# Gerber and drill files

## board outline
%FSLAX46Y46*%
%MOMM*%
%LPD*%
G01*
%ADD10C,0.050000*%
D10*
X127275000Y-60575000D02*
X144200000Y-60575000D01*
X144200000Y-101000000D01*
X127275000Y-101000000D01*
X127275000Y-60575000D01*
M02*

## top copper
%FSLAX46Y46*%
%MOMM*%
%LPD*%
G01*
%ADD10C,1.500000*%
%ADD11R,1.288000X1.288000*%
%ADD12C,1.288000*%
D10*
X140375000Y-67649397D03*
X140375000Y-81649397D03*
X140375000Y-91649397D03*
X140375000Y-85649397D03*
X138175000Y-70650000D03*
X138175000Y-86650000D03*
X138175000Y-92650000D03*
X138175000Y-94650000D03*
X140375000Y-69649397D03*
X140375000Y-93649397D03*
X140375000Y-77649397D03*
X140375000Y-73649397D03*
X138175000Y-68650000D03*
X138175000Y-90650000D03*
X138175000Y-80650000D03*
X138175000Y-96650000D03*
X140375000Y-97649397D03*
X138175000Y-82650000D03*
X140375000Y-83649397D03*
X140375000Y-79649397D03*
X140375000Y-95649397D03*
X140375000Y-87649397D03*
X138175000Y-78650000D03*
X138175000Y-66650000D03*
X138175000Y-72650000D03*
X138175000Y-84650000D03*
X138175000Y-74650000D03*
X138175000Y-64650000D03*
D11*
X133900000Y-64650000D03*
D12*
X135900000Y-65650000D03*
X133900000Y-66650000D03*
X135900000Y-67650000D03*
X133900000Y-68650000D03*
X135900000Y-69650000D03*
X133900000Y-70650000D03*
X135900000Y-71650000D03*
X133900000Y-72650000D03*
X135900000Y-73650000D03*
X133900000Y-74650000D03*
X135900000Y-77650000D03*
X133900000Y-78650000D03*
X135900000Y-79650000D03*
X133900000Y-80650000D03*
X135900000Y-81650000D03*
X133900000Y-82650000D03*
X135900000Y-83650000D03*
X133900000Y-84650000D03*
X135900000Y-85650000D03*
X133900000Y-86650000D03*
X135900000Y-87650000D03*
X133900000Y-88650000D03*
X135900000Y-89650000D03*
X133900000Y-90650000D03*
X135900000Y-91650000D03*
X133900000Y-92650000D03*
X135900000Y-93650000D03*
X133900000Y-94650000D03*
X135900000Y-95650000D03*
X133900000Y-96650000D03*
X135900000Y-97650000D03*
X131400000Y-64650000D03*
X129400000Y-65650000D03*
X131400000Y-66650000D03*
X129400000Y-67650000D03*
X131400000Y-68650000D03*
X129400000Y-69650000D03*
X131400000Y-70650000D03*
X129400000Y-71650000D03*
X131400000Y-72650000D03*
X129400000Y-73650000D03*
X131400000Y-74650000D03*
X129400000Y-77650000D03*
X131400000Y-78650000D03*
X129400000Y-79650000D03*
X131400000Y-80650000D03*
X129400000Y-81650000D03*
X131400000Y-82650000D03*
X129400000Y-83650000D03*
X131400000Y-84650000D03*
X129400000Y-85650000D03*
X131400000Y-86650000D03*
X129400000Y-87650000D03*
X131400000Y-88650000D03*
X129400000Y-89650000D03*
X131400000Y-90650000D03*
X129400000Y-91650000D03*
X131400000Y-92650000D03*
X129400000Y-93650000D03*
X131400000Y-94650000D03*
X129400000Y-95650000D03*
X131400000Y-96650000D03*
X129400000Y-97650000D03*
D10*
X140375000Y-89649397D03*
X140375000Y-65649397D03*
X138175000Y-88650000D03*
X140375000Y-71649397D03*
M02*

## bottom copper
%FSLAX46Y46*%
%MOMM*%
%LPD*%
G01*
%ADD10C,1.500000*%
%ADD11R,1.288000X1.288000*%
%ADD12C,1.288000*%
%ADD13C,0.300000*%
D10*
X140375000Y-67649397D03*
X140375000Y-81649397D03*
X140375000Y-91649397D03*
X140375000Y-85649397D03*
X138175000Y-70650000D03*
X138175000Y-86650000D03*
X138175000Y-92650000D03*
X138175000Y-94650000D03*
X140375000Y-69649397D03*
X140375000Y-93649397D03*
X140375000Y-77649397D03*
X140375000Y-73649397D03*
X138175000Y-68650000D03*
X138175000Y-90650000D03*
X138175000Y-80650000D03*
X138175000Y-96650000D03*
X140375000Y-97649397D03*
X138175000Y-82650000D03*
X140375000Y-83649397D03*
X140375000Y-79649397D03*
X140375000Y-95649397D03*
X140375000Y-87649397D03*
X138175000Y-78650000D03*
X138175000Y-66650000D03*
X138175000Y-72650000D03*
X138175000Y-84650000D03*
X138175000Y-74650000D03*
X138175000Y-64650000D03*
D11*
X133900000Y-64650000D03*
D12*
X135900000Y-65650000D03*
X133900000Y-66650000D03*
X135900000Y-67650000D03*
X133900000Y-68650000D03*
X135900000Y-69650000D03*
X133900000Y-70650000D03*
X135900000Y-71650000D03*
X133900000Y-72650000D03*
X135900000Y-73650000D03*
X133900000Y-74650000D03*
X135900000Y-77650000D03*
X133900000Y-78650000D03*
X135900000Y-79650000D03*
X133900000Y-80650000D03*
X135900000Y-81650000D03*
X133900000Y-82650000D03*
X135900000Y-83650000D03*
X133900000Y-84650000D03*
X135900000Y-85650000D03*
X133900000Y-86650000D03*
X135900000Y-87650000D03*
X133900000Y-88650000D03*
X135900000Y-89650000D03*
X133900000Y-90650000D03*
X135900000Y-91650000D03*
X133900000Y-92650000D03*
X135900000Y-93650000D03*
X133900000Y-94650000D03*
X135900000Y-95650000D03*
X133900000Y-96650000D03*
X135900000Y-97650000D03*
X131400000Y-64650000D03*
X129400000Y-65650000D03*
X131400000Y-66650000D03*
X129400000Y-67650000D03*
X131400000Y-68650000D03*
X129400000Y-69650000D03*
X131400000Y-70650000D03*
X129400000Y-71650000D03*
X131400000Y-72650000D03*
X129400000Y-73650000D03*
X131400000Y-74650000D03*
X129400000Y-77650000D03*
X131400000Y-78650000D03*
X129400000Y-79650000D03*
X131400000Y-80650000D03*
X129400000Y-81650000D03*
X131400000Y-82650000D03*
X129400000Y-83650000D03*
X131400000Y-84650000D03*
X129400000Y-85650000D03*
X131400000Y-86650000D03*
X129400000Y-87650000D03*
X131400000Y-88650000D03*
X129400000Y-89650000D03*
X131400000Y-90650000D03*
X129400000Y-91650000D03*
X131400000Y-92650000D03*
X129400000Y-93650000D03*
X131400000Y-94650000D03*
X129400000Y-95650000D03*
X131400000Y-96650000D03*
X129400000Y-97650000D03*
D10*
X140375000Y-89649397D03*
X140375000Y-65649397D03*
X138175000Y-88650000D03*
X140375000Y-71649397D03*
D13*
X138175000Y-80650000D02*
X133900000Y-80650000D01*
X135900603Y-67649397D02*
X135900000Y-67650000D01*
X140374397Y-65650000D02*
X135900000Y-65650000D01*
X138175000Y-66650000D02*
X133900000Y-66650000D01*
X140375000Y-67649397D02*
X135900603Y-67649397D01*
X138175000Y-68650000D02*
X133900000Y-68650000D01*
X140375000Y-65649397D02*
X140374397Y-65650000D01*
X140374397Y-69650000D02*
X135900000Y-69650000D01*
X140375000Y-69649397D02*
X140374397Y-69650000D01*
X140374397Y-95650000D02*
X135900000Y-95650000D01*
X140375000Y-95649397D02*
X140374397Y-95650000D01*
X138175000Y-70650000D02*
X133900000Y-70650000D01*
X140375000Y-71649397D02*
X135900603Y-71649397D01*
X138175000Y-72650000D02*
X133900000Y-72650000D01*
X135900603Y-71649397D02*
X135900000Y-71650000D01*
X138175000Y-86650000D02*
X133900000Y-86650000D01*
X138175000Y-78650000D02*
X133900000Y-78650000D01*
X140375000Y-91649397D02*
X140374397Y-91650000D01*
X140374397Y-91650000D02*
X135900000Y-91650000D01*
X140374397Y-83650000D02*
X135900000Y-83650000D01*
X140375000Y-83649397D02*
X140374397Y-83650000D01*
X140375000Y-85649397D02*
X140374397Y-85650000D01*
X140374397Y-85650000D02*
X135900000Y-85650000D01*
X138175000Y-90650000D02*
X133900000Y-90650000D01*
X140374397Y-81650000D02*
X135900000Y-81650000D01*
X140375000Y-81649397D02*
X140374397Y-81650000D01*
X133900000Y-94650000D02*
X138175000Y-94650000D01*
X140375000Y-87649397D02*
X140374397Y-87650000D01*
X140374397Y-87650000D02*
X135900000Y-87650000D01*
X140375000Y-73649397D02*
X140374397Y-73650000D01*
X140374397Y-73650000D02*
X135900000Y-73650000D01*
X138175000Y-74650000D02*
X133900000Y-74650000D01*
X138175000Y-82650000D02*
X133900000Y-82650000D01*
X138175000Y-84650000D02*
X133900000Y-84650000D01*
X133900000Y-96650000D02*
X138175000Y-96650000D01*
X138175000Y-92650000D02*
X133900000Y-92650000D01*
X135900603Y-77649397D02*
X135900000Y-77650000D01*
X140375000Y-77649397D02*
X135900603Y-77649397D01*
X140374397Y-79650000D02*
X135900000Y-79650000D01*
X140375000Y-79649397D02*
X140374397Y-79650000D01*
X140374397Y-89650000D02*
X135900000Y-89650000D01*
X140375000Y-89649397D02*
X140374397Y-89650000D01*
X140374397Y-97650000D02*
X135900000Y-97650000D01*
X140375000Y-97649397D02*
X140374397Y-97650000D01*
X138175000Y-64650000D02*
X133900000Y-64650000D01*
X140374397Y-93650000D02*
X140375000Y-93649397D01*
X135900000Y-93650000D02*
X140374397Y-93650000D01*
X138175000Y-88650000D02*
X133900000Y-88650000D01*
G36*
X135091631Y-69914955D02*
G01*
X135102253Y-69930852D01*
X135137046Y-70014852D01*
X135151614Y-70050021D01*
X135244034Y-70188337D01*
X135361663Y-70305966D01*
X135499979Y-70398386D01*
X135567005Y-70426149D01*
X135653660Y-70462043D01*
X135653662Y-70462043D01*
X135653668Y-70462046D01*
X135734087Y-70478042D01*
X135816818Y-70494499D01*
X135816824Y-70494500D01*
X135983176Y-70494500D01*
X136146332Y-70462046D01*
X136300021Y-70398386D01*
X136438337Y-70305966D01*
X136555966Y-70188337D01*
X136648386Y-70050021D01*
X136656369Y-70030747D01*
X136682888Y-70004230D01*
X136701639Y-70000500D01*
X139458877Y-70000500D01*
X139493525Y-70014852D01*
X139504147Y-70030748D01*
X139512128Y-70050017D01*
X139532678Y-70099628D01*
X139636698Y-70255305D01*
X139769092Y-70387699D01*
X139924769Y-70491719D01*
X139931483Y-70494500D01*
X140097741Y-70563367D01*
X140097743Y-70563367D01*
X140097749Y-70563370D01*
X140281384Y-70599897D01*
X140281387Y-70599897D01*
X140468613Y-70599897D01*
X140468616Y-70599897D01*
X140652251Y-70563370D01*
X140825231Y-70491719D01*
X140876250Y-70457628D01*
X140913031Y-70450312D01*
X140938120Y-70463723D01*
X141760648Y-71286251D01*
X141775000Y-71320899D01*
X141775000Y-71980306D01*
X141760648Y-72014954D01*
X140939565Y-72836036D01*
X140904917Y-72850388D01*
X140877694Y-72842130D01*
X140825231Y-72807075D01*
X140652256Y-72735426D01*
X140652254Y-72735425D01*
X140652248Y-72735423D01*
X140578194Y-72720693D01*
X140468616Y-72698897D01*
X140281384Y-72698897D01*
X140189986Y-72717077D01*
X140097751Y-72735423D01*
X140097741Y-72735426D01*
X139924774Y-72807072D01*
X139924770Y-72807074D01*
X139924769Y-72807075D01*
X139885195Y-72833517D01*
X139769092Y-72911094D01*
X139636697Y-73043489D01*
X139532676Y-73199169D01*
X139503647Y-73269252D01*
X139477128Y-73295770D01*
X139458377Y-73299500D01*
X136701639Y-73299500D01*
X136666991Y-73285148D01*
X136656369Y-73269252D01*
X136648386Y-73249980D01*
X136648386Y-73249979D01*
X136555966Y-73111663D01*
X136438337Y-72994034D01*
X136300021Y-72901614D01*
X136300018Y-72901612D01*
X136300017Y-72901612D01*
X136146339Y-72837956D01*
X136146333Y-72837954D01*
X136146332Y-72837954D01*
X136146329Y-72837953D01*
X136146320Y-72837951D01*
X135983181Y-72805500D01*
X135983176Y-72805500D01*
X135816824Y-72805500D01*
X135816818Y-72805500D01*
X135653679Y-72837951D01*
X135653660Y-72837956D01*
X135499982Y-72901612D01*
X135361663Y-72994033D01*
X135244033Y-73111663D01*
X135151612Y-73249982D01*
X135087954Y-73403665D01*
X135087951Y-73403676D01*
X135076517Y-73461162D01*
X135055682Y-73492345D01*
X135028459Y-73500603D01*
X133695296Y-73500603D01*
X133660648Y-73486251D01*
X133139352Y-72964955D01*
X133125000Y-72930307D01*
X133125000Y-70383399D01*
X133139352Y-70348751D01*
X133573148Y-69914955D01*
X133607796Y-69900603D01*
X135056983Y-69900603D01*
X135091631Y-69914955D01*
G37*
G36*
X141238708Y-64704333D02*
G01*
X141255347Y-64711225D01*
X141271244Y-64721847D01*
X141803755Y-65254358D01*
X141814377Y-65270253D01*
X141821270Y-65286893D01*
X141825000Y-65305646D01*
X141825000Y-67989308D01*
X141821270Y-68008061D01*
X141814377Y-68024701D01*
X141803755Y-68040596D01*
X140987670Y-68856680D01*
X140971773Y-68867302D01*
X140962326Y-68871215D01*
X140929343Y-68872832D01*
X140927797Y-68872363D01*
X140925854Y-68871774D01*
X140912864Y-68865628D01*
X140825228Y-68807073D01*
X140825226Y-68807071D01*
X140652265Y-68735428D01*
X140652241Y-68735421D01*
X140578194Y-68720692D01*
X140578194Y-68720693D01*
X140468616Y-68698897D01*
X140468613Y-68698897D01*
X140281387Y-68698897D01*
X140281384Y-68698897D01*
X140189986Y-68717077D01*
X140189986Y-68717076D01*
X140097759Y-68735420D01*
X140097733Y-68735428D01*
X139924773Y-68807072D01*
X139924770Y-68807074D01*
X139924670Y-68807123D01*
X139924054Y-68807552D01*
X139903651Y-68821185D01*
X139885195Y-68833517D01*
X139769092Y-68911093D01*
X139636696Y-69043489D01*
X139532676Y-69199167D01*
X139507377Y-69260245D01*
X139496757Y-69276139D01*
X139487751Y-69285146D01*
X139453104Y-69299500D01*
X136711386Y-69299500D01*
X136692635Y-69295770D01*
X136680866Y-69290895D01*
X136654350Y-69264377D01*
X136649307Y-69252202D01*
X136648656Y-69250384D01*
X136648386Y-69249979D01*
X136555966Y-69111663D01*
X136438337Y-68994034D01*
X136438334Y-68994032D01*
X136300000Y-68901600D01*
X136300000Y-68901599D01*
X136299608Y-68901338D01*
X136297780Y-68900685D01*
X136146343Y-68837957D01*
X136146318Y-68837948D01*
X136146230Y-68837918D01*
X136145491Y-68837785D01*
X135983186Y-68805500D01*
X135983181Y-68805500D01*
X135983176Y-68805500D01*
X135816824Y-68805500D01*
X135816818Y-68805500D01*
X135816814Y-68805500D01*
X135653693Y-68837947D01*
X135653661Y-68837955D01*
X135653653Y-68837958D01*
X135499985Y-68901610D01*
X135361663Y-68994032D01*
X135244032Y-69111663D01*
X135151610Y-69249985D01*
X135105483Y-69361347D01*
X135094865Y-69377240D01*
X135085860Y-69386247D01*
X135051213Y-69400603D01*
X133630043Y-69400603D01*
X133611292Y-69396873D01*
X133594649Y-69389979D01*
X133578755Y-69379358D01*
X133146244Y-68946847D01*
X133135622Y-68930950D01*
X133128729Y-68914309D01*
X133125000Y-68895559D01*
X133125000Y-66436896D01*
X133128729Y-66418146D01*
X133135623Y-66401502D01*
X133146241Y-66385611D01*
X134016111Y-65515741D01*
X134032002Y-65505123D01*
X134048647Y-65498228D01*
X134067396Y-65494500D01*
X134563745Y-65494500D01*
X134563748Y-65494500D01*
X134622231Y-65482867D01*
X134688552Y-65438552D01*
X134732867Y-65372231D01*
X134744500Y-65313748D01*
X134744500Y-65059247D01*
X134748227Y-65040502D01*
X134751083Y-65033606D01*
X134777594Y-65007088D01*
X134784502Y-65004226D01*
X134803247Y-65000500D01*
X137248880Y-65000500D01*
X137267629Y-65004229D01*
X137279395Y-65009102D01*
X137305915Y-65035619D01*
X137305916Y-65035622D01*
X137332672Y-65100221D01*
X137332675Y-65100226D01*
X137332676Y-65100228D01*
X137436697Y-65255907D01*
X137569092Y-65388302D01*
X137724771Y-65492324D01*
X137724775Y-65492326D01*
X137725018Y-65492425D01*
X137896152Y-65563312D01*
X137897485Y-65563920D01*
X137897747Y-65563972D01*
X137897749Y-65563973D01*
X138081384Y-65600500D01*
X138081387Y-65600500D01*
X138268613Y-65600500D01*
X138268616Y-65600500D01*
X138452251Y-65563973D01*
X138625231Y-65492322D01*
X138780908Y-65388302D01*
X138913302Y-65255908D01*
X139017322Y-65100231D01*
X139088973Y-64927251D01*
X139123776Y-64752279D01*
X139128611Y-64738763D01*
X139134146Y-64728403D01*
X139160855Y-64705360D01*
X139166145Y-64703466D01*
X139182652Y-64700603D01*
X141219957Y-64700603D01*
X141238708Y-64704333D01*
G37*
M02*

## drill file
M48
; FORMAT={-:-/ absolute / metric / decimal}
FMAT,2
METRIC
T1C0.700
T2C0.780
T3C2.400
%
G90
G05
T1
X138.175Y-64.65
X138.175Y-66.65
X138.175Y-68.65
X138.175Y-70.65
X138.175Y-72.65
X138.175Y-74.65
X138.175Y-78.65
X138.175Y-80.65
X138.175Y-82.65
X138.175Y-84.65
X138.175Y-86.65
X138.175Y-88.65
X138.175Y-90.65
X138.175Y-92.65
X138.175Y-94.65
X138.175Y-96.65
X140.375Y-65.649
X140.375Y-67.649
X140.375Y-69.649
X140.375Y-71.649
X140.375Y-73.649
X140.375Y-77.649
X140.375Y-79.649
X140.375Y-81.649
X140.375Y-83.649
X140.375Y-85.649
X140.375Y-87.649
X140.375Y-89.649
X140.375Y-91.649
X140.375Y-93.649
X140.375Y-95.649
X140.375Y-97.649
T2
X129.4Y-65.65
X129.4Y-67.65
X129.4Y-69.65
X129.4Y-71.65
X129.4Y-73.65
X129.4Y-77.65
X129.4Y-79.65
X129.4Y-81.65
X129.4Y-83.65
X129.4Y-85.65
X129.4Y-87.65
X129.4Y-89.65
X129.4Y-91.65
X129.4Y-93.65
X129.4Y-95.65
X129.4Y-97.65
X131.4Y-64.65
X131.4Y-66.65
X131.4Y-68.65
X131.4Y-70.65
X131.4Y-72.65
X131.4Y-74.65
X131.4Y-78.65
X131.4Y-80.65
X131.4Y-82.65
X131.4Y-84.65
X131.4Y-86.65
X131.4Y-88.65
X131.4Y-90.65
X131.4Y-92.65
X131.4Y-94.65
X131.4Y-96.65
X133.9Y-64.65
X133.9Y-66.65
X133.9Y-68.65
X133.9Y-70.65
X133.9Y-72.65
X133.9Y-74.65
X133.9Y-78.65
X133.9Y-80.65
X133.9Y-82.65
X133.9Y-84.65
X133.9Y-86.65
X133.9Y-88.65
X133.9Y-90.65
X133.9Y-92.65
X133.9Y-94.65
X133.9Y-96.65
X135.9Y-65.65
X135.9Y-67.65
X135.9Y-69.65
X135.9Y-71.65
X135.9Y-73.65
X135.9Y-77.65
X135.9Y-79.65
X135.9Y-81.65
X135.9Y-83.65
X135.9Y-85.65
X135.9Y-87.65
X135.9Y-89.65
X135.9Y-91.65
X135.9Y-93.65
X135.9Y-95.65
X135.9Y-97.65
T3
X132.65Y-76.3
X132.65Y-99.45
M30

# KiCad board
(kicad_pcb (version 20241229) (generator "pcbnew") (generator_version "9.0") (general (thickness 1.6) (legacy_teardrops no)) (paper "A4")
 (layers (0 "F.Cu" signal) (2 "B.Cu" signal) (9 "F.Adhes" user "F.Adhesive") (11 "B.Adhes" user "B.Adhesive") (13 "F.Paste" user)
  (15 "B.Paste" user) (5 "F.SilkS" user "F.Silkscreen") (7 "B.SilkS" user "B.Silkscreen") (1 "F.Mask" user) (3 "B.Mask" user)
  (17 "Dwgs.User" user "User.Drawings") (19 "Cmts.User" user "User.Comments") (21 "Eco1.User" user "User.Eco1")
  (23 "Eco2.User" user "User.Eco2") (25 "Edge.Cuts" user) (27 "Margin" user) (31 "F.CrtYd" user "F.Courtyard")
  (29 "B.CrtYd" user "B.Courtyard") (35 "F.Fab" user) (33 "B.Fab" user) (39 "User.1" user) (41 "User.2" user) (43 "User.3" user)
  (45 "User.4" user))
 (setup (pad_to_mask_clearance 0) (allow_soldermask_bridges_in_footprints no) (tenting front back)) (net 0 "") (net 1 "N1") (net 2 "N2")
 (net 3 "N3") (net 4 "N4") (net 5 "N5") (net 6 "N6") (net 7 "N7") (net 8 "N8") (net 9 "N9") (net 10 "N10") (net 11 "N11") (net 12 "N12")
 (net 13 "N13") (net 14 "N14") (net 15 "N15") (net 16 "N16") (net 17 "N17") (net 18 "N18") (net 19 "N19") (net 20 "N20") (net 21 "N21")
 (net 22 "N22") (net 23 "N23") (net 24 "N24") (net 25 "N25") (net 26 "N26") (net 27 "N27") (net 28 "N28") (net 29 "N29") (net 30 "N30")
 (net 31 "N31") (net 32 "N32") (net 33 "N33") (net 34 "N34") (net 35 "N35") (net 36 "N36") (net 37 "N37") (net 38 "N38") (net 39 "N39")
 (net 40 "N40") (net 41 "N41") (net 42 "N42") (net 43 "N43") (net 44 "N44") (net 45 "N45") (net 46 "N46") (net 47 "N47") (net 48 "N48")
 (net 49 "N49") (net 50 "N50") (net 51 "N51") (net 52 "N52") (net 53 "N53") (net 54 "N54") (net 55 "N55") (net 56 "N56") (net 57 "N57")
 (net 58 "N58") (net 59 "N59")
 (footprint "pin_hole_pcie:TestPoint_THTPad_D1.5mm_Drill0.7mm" (layer "F.Cu") (at 140.375 67.649397 180)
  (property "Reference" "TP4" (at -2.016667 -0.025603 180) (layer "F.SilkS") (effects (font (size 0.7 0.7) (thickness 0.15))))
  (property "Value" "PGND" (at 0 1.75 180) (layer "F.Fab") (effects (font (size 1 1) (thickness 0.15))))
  (pad "1" thru_hole circle (at 0 0 180) (size 1.5 1.5) (drill 0.7) (layers "*.Cu" "*.Mask") (remove_unused_layers no) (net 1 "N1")))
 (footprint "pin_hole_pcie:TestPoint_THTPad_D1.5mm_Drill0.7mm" (layer "F.Cu") (at 140.375 81.649397 180)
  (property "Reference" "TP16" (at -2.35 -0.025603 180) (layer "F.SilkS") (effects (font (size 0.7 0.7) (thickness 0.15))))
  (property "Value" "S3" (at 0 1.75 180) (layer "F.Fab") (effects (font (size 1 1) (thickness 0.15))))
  (pad "1" thru_hole circle (at 0 0 180) (size 1.5 1.5) (drill 0.7) (layers "*.Cu" "*.Mask") (remove_unused_layers no) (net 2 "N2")))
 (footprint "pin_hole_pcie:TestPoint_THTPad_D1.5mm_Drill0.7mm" (layer "F.Cu") (at 140.375 91.649397 180)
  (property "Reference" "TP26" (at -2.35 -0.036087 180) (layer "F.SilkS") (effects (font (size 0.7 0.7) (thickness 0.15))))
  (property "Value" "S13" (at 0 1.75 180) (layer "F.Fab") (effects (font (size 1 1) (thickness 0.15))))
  (pad "1" thru_hole circle (at 0 0 180) (size 1.5 1.5) (drill 0.7) (layers "*.Cu" "*.Mask") (remove_unused_layers no) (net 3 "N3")))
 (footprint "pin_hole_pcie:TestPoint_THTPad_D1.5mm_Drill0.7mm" (layer "F.Cu") (at 140.375 85.649397 180)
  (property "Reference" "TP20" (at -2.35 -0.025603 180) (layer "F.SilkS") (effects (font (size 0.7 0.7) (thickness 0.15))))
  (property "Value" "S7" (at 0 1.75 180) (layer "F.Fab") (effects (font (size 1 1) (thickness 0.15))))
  (pad "1" thru_hole circle (at 0 0 180) (size 1.5 1.5) (drill 0.7) (layers "*.Cu" "*.Mask") (remove_unused_layers no) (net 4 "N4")))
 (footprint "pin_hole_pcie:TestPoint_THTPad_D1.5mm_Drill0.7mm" (layer "F.Cu") (at 138.175 70.65 180)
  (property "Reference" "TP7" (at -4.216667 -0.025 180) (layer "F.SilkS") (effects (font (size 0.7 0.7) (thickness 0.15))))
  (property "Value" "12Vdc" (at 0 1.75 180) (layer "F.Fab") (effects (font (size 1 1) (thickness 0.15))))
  (pad "1" thru_hole circle (at 0 0 180) (size 1.5 1.5) (drill 0.7) (layers "*.Cu" "*.Mask") (remove_unused_layers no) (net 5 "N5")))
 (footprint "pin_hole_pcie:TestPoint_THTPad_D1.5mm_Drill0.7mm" (layer "F.Cu") (at 138.175 86.65 180)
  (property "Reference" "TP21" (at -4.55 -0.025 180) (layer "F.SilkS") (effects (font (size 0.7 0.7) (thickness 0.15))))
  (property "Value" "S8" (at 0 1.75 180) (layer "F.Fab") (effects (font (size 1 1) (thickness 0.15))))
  (pad "1" thru_hole circle (at 0 0 180) (size 1.5 1.5) (drill 0.7) (layers "*.Cu" "*.Mask") (remove_unused_layers no) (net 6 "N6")))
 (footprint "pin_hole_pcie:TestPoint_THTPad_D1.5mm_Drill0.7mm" (layer "F.Cu") (at 138.175 92.65 180)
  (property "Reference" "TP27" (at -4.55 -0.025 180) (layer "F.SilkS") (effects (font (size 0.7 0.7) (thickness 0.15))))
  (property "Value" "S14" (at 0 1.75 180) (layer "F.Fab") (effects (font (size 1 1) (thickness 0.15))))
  (pad "1" thru_hole circle (at 0 0 180) (size 1.5 1.5) (drill 0.7) (layers "*.Cu" "*.Mask") (remove_unused_layers no) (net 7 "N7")))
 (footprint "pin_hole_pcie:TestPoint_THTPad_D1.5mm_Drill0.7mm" (layer "F.Cu") (at 138.175 94.65 180)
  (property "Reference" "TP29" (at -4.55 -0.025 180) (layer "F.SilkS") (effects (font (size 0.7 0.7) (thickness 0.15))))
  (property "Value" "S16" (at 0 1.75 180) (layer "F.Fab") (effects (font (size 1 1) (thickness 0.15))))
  (pad "1" thru_hole circle (at 0 0 180) (size 1.5 1.5) (drill 0.7) (layers "*.Cu" "*.Mask") (remove_unused_layers no) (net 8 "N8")))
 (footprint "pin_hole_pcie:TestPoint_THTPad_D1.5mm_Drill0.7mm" (layer "F.Cu") (at 140.375 69.649397 180)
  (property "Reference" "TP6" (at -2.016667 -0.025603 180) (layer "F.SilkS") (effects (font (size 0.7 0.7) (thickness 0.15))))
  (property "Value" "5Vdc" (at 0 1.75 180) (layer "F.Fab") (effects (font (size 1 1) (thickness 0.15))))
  (pad "1" thru_hole circle (at 0 0 180) (size 1.5 1.5) (drill 0.7) (layers "*.Cu" "*.Mask") (remove_unused_layers no) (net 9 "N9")))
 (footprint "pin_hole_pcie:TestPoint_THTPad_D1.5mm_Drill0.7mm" (layer "F.Cu") (at 140.375 93.649397 180)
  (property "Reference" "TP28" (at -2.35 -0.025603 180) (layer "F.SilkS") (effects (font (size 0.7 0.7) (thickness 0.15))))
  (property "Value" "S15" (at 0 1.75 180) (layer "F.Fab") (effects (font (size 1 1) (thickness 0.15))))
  (pad "1" thru_hole circle (at 0 0 180) (size 1.5 1.5) (drill 0.7) (layers "*.Cu" "*.Mask") (remove_unused_layers no) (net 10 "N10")))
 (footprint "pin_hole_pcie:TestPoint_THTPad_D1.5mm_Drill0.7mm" (layer "F.Cu") (at 140.375 77.649397 180)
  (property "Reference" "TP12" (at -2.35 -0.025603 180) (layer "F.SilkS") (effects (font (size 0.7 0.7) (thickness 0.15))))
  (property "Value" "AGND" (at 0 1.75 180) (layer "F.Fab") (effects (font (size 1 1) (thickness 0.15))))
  (pad "1" thru_hole circle (at 0 0 180) (size 1.5 1.5) (drill 0.7) (layers "*.Cu" "*.Mask") (remove_unused_layers no) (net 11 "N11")))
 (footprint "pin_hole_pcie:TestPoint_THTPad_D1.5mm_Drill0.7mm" (layer "F.Cu") (at 140.375 73.649397 180)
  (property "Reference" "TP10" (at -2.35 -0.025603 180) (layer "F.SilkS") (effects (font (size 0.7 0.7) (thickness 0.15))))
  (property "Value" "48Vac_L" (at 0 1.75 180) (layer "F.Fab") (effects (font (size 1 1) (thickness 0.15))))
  (pad "1" thru_hole circle (at 0 0 180) (size 1.5 1.5) (drill 0.7) (layers "*.Cu" "*.Mask") (remove_unused_layers no) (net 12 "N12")))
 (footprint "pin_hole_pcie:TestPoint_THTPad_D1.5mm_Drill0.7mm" (layer "F.Cu") (at 138.175 68.65 180)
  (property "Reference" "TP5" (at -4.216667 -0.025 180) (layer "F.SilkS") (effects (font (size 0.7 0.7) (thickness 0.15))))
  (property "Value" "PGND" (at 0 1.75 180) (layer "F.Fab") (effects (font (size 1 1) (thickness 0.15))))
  (pad "1" thru_hole circle (at 0 0 180) (size 1.5 1.5) (drill 0.7) (layers "*.Cu" "*.Mask") (remove_unused_layers no) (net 1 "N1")))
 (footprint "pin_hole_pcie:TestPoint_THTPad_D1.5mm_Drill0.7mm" (layer "F.Cu") (at 138.175 90.65 180)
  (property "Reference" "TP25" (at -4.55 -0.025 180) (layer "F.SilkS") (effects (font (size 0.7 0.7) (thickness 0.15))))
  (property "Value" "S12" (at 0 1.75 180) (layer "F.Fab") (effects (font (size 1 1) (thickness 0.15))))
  (pad "1" thru_hole circle (at 0 0 180) (size 1.5 1.5) (drill 0.7) (layers "*.Cu" "*.Mask") (remove_unused_layers no) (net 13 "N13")))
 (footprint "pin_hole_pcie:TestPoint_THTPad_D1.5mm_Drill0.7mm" (layer "F.Cu") (at 138.175 80.65 180)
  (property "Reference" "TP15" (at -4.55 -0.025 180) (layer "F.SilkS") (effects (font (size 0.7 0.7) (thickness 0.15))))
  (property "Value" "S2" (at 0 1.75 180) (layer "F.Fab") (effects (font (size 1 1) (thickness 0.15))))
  (pad "1" thru_hole circle (at 0 0 180) (size 1.5 1.5) (drill 0.7) (layers "*.Cu" "*.Mask") (remove_unused_layers no) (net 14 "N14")))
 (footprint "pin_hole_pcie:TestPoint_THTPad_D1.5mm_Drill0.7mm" (layer "F.Cu") (at 138.175 96.65 180)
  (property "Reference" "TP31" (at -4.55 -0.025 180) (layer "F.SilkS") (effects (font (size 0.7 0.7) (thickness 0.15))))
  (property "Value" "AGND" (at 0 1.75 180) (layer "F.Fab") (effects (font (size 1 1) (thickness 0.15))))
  (pad "1" thru_hole circle (at 0 0 180) (size 1.5 1.5) (drill 0.7) (layers "*.Cu" "*.Mask") (remove_unused_layers no) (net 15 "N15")))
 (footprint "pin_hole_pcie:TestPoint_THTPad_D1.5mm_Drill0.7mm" (layer "F.Cu") (at 140.375 97.649397 180)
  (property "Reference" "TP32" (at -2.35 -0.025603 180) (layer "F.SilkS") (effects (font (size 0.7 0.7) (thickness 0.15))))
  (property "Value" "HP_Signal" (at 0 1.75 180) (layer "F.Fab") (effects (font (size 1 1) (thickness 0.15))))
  (pad "1" thru_hole circle (at 0 0 180) (size 1.5 1.5) (drill 0.7) (layers "*.Cu" "*.Mask") (remove_unused_layers no) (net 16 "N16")))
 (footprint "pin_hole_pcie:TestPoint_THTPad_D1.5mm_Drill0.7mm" (layer "F.Cu") (at 138.175 82.65 180)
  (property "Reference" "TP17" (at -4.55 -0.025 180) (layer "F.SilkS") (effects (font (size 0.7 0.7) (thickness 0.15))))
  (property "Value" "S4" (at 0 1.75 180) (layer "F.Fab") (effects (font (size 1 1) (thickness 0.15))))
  (pad "1" thru_hole circle (at 0 0 180) (size 1.5 1.5) (drill 0.7) (layers "*.Cu" "*.Mask") (remove_unused_layers no) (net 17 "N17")))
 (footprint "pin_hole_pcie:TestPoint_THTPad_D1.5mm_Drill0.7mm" (layer "F.Cu") (at 140.375 83.649397 180)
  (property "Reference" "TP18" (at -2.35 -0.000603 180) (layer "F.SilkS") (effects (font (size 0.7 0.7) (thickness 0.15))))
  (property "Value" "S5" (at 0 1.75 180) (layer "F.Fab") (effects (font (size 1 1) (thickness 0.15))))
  (pad "1" thru_hole circle (at 0 0 180) (size 1.5 1.5) (drill 0.7) (layers "*.Cu" "*.Mask") (remove_unused_layers no) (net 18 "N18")))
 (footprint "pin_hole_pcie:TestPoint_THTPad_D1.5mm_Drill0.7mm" (layer "F.Cu") (at 140.375 79.649397 180)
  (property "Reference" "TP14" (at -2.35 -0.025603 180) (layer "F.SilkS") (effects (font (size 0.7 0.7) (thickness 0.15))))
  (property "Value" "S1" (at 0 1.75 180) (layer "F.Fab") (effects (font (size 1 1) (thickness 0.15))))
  (pad "1" thru_hole circle (at 0 0 180) (size 1.5 1.5) (drill 0.7) (layers "*.Cu" "*.Mask") (remove_unused_layers no) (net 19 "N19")))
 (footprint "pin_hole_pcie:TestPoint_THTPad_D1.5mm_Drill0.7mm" (layer "F.Cu") (at 140.375 95.649397 180)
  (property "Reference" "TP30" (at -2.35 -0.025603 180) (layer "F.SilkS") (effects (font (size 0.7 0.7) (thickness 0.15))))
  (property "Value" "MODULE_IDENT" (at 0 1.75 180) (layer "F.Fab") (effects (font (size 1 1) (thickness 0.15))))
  (pad "1" thru_hole circle (at 0 0 180) (size 1.5 1.5) (drill 0.7) (layers "*.Cu" "*.Mask") (remove_unused_layers no) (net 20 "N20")))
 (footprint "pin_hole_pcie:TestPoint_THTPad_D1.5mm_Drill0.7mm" (layer "F.Cu") (at 140.375 87.649397 180)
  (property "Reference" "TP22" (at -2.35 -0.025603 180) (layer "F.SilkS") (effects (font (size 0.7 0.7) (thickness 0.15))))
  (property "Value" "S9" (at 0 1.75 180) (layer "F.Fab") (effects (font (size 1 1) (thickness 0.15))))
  (pad "1" thru_hole circle (at 0 0 180) (size 1.5 1.5) (drill 0.7) (layers "*.Cu" "*.Mask") (remove_unused_layers no) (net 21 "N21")))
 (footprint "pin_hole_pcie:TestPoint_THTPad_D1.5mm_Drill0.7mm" (layer "F.Cu") (at 138.175 78.65 180)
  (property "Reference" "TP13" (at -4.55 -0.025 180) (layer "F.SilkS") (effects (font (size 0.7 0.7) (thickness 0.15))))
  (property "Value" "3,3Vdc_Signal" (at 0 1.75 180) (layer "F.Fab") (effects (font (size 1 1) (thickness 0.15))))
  (pad "1" thru_hole circle (at 0 0 180) (size 1.5 1.5) (drill 0.7) (layers "*.Cu" "*.Mask") (remove_unused_layers no) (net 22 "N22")))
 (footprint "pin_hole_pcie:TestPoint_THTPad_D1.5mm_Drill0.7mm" (layer "F.Cu") (at 138.175 66.65 180)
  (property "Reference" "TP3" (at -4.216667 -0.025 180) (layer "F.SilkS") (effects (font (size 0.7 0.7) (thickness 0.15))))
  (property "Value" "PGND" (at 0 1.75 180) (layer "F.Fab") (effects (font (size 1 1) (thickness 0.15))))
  (pad "1" thru_hole circle (at 0 0 180) (size 1.5 1.5) (drill 0.7) (layers "*.Cu" "*.Mask") (remove_unused_layers no) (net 1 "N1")))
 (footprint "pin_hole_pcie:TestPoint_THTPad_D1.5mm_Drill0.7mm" (layer "F.Cu") (at 138.175 72.65 180)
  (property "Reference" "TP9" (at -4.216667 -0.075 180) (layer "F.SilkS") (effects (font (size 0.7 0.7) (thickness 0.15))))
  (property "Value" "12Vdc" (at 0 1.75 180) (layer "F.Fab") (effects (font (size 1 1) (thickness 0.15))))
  (pad "1" thru_hole circle (at 0 0 180) (size 1.5 1.5) (drill 0.7) (layers "*.Cu" "*.Mask") (remove_unused_layers no) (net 5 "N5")))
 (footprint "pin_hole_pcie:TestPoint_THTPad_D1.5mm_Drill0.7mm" (layer "F.Cu") (at 138.175 84.65 180)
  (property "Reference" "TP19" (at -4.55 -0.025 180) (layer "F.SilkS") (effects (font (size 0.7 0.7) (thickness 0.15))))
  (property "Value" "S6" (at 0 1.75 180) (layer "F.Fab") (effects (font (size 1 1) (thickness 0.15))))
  (pad "1" thru_hole circle (at 0 0 180) (size 1.5 1.5) (drill 0.7) (layers "*.Cu" "*.Mask") (remove_unused_layers no) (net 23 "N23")))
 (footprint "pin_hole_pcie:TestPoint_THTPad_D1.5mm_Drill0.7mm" (layer "F.Cu") (at 138.175 74.65 180)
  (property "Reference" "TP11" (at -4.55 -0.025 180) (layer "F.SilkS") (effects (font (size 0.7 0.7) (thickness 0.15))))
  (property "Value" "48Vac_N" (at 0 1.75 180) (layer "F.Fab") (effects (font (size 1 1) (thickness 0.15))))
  (pad "1" thru_hole circle (at 0 0 180) (size 1.5 1.5) (drill 0.7) (layers "*.Cu" "*.Mask") (remove_unused_layers no) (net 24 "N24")))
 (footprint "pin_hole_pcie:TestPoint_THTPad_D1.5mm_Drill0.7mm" (layer "F.Cu") (at 138.175 64.65 180)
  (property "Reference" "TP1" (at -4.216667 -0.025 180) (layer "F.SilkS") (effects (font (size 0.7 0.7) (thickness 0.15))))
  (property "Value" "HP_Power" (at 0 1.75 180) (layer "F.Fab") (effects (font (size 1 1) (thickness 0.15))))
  (pad "1" thru_hole circle (at 0 0 180) (size 1.5 1.5) (drill 0.7) (layers "*.Cu" "*.Mask") (remove_unused_layers no) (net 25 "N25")))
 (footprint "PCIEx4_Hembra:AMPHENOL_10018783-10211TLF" (layer "F.Cu") (at 132.65 76.3 -90)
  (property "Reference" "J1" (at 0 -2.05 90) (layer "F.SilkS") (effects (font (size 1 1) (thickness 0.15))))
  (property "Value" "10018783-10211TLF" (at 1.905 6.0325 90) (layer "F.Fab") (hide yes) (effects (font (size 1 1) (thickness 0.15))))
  (pad "" np_thru_hole circle (at 0 0 270) (size 2.4 2.4) (drill 2.4) (layers "*.Cu" "*.Mask"))
  (pad "" np_thru_hole circle (at 23.15 0 270) (size 2.4 2.4) (drill 2.4) (layers "*.Cu" "*.Mask"))
  (pad "A1" thru_hole rect (at -11.65 -1.25 270) (size 1.288 1.288) (drill 0.78) (layers "*.Cu" "*.Mask") (remove_unused_layers no)
   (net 25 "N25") (solder_mask_margin 0.102))
  (pad "A2" thru_hole circle (at -10.65 -3.25 270) (size 1.288 1.288) (drill 0.78) (layers "*.Cu" "*.Mask") (remove_unused_layers no)
   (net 1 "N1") (solder_mask_margin 0.102))
  (pad "A3" thru_hole circle (at -9.65 -1.25 270) (size 1.288 1.288) (drill 0.78) (layers "*.Cu" "*.Mask") (remove_unused_layers no)
   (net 1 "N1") (solder_mask_margin 0.102))
  (pad "A4" thru_hole circle (at -8.65 -3.25 270) (size 1.288 1.288) (drill 0.78) (layers "*.Cu" "*.Mask") (remove_unused_layers no)
   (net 1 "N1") (solder_mask_margin 0.102))
  (pad "A5" thru_hole circle (at -7.65 -1.25 270) (size 1.288 1.288) (drill 0.78) (layers "*.Cu" "*.Mask") (remove_unused_layers no)
   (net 1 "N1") (solder_mask_margin 0.102))
  (pad "A6" thru_hole circle (at -6.65 -3.25 270) (size 1.288 1.288) (drill 0.78) (layers "*.Cu" "*.Mask") (remove_unused_layers no)
   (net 9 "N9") (solder_mask_margin 0.102))
  (pad "A7" thru_hole circle (at -5.65 -1.25 270) (size 1.288 1.288) (drill 0.78) (layers "*.Cu" "*.Mask") (remove_unused_layers no)
   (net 5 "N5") (solder_mask_margin 0.102))
  (pad "A8" thru_hole circle (at -4.65 -3.25 270) (size 1.288 1.288) (drill 0.78) (layers "*.Cu" "*.Mask") (remove_unused_layers no)
   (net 5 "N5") (solder_mask_margin 0.102))
  (pad "A9" thru_hole circle (at -3.65 -1.25 270) (size 1.288 1.288) (drill 0.78) (layers "*.Cu" "*.Mask") (remove_unused_layers no)
   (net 5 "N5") (solder_mask_margin 0.102))
  (pad "A10" thru_hole circle (at -2.65 -3.25 270) (size 1.288 1.288) (drill 0.78) (layers "*.Cu" "*.Mask") (remove_unused_layers no)
   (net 12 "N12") (solder_mask_margin 0.102))
  (pad "A11" thru_hole circle (at -1.65 -1.25 270) (size 1.288 1.288) (drill 0.78) (layers "*.Cu" "*.Mask") (remove_unused_layers no)
   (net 24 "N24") (solder_mask_margin 0.102))
  (pad "A12" thru_hole circle (at 1.35 -3.25 270) (size 1.288 1.288) (drill 0.78) (layers "*.Cu" "*.Mask") (remove_unused_layers no)
   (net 11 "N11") (solder_mask_margin 0.102))
  (pad "A13" thru_hole circle (at 2.35 -1.25 270) (size 1.288 1.288) (drill 0.78) (layers "*.Cu" "*.Mask") (remove_unused_layers no)
   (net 22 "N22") (solder_mask_margin 0.102))
  (pad "A14" thru_hole circle (at 3.35 -3.25 270) (size 1.288 1.288) (drill 0.78) (layers "*.Cu" "*.Mask") (remove_unused_layers no)
   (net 19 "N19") (solder_mask_margin 0.102))
  (pad "A15" thru_hole circle (at 4.35 -1.25 270) (size 1.288 1.288) (drill 0.78) (layers "*.Cu" "*.Mask") (remove_unused_layers no)
   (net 14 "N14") (solder_mask_margin 0.102))
  (pad "A16" thru_hole circle (at 5.35 -3.25 270) (size 1.288 1.288) (drill 0.78) (layers "*.Cu" "*.Mask") (remove_unused_layers no)
   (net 2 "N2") (solder_mask_margin 0.102))
  (pad "A17" thru_hole circle (at 6.35 -1.25 270) (size 1.288 1.288) (drill 0.78) (layers "*.Cu" "*.Mask") (remove_unused_layers no)
   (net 17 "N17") (solder_mask_margin 0.102))
  (pad "A18" thru_hole circle (at 7.35 -3.25 270) (size 1.288 1.288) (drill 0.78) (layers "*.Cu" "*.Mask") (remove_unused_layers no)
   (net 18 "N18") (solder_mask_margin 0.102))
  (pad "A19" thru_hole circle (at 8.35 -1.25 270) (size 1.288 1.288) (drill 0.78) (layers "*.Cu" "*.Mask") (remove_unused_layers no)
   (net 23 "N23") (solder_mask_margin 0.102))
  (pad "A20" thru_hole circle (at 9.35 -3.25 270) (size 1.288 1.288) (drill 0.78) (layers "*.Cu" "*.Mask") (remove_unused_layers no)
   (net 4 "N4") (solder_mask_margin 0.102))
  (pad "A21" thru_hole circle (at 10.35 -1.25 270) (size 1.288 1.288) (drill 0.78) (layers "*.Cu" "*.Mask") (remove_unused_layers no)
   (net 6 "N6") (solder_mask_margin 0.102))
  (pad "A22" thru_hole circle (at 11.35 -3.25 270) (size 1.288 1.288) (drill 0.78) (layers "*.Cu" "*.Mask") (remove_unused_layers no)
   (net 21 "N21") (solder_mask_margin 0.102))
  (pad "A23" thru_hole circle (at 12.35 -1.25 270) (size 1.288 1.288) (drill 0.78) (layers "*.Cu" "*.Mask") (remove_unused_layers no)
   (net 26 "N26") (solder_mask_margin 0.102))
  (pad "A24" thru_hole circle (at 13.35 -3.25 270) (size 1.288 1.288) (drill 0.78) (layers "*.Cu" "*.Mask") (remove_unused_layers no)
   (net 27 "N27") (solder_mask_margin 0.102))
  (pad "A25" thru_hole circle (at 14.35 -1.25 270) (size 1.288 1.288) (drill 0.78) (layers "*.Cu" "*.Mask") (remove_unused_layers no)
   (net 13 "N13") (solder_mask_margin 0.102))
  (pad "A26" thru_hole circle (at 15.35 -3.25 270) (size 1.288 1.288) (drill 0.78) (layers "*.Cu" "*.Mask") (remove_unused_layers no)
   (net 3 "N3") (solder_mask_margin 0.102))
  (pad "A27" thru_hole circle (at 16.35 -1.25 270) (size 1.288 1.288) (drill 0.78) (layers "*.Cu" "*.Mask") (remove_unused_layers no)
   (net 7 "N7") (solder_mask_margin 0.102))
  (pad "A28" thru_hole circle (at 17.35 -3.25 270) (size 1.288 1.288) (drill 0.78) (layers "*.Cu" "*.Mask") (remove_unused_layers no)
   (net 10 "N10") (solder_mask_margin 0.102))
  (pad "A29" thru_hole circle (at 18.35 -1.25 270) (size 1.288 1.288) (drill 0.78) (layers "*.Cu" "*.Mask") (remove_unused_layers no)
   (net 8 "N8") (solder_mask_margin 0.102))
  (pad "A30" thru_hole circle (at 19.35 -3.25 270) (size 1.288 1.288) (drill 0.78) (layers "*.Cu" "*.Mask") (remove_unused_layers no)
   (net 20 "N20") (solder_mask_margin 0.102))
  (pad "A31" thru_hole circle (at 20.35 -1.25 270) (size 1.288 1.288) (drill 0.78) (layers "*.Cu" "*.Mask") (remove_unused_layers no)
   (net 15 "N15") (solder_mask_margin 0.102))
  (pad "A32" thru_hole circle (at 21.35 -3.25 270) (size 1.288 1.288) (drill 0.78) (layers "*.Cu" "*.Mask") (remove_unused_layers no)
   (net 16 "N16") (solder_mask_margin 0.102))
  (pad "B1" thru_hole circle (at -11.65 1.25 270) (size 1.288 1.288) (drill 0.78) (layers "*.Cu" "*.Mask") (remove_unused_layers no)
   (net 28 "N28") (solder_mask_margin 0.102))
  (pad "B2" thru_hole circle (at -10.65 3.25 270) (size 1.288 1.288) (drill 0.78) (layers "*.Cu" "*.Mask") (remove_unused_layers no)
   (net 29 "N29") (solder_mask_margin 0.102))
  (pad "B3" thru_hole circle (at -9.65 1.25 270) (size 1.288 1.288) (drill 0.78) (layers "*.Cu" "*.Mask") (remove_unused_layers no)
   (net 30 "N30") (solder_mask_margin 0.102))
  (pad "B4" thru_hole circle (at -8.65 3.25 270) (size 1.288 1.288) (drill 0.78) (layers "*.Cu" "*.Mask") (remove_unused_layers no)
   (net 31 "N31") (solder_mask_margin 0.102))
  (pad "B5" thru_hole circle (at -7.65 1.25 270) (size 1.288 1.288) (drill 0.78) (layers "*.Cu" "*.Mask") (remove_unused_layers no)
   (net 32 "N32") (solder_mask_margin 0.102))
  (pad "B6" thru_hole circle (at -6.65 3.25 270) (size 1.288 1.288) (drill 0.78) (layers "*.Cu" "*.Mask") (remove_unused_layers no)
   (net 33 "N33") (solder_mask_margin 0.102))
  (pad "B7" thru_hole circle (at -5.65 1.25 270) (size 1.288 1.288) (drill 0.78) (layers "*.Cu" "*.Mask") (remove_unused_layers no)
   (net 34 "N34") (solder_mask_margin 0.102))
  (pad "B8" thru_hole circle (at -4.65 3.25 270) (size 1.288 1.288) (drill 0.78) (layers "*.Cu" "*.Mask") (remove_unused_layers no)
   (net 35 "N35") (solder_mask_margin 0.102))
  (pad "B9" thru_hole circle (at -3.65 1.25 270) (size 1.288 1.288) (drill 0.78) (layers "*.Cu" "*.Mask") (remove_unused_layers no)
   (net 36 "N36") (solder_mask_margin 0.102))
  (pad "B10" thru_hole circle (at -2.65 3.25 270) (size 1.288 1.288) (drill 0.78) (layers "*.Cu" "*.Mask") (remove_unused_layers no)
   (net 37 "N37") (solder_mask_margin 0.102))
  (pad "B11" thru_hole circle (at -1.65 1.25 270) (size 1.288 1.288) (drill 0.78) (layers "*.Cu" "*.Mask") (remove_unused_layers no)
   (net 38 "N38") (solder_mask_margin 0.102))
  (pad "B12" thru_hole circle (at 1.35 3.25 270) (size 1.288 1.288) (drill 0.78) (layers "*.Cu" "*.Mask") (remove_unused_layers no)
   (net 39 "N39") (solder_mask_margin 0.102))
  (pad "B13" thru_hole circle (at 2.35 1.25 270) (size 1.288 1.288) (drill 0.78) (layers "*.Cu" "*.Mask") (remove_unused_layers no)
   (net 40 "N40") (solder_mask_margin 0.102))
  (pad "B14" thru_hole circle (at 3.35 3.25 270) (size 1.288 1.288) (drill 0.78) (layers "*.Cu" "*.Mask") (remove_unused_layers no)
   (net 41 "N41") (solder_mask_margin 0.102))
  (pad "B15" thru_hole circle (at 4.35 1.25 270) (size 1.288 1.288) (drill 0.78) (layers "*.Cu" "*.Mask") (remove_unused_layers no)
   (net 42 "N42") (solder_mask_margin 0.102))
  (pad "B16" thru_hole circle (at 5.35 3.25 270) (size 1.288 1.288) (drill 0.78) (layers "*.Cu" "*.Mask") (remove_unused_layers no)
   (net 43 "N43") (solder_mask_margin 0.102))
  (pad "B17" thru_hole circle (at 6.35 1.25 270) (size 1.288 1.288) (drill 0.78) (layers "*.Cu" "*.Mask") (remove_unused_layers no)
   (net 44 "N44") (solder_mask_margin 0.102))
  (pad "B18" thru_hole circle (at 7.35 3.25 270) (size 1.288 1.288) (drill 0.78) (layers "*.Cu" "*.Mask") (remove_unused_layers no)
   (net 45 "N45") (solder_mask_margin 0.102))
  (pad "B19" thru_hole circle (at 8.35 1.25 270) (size 1.288 1.288) (drill 0.78) (layers "*.Cu" "*.Mask") (remove_unused_layers no)
   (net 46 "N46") (solder_mask_margin 0.102))
  (pad "B20" thru_hole circle (at 9.35 3.25 270) (size 1.288 1.288) (drill 0.78) (layers "*.Cu" "*.Mask") (remove_unused_layers no)
   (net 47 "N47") (solder_mask_margin 0.102))
  (pad "B21" thru_hole circle (at 10.35 1.25 270) (size 1.288 1.288) (drill 0.78) (layers "*.Cu" "*.Mask") (remove_unused_layers no)
   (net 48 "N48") (solder_mask_margin 0.102))
  (pad "B22" thru_hole circle (at 11.35 3.25 270) (size 1.288 1.288) (drill 0.78) (layers "*.Cu" "*.Mask") (remove_unused_layers no)
   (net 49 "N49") (solder_mask_margin 0.102))
  (pad "B23" thru_hole circle (at 12.35 1.25 270) (size 1.288 1.288) (drill 0.78) (layers "*.Cu" "*.Mask") (remove_unused_layers no)
   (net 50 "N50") (solder_mask_margin 0.102))
  (pad "B24" thru_hole circle (at 13.35 3.25 270) (size 1.288 1.288) (drill 0.78) (layers "*.Cu" "*.Mask") (remove_unused_layers no)
   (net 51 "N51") (solder_mask_margin 0.102))
  (pad "B25" thru_hole circle (at 14.35 1.25 270) (size 1.288 1.288) (drill 0.78) (layers "*.Cu" "*.Mask") (remove_unused_layers no)
   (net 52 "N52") (solder_mask_margin 0.102))
  (pad "B26" thru_hole circle (at 15.35 3.25 270) (size 1.288 1.288) (drill 0.78) (layers "*.Cu" "*.Mask") (remove_unused_layers no)
   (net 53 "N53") (solder_mask_margin 0.102))
  (pad "B27" thru_hole circle (at 16.35 1.25 270) (size 1.288 1.288) (drill 0.78) (layers "*.Cu" "*.Mask") (remove_unused_layers no)
   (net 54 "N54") (solder_mask_margin 0.102))
  (pad "B28" thru_hole circle (at 17.35 3.25 270) (size 1.288 1.288) (drill 0.78) (layers "*.Cu" "*.Mask") (remove_unused_layers no)
   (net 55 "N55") (solder_mask_margin 0.102))
  (pad "B29" thru_hole circle (at 18.35 1.25 270) (size 1.288 1.288) (drill 0.78) (layers "*.Cu" "*.Mask") (remove_unused_layers no)
   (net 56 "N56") (solder_mask_margin 0.102))
  (pad "B30" thru_hole circle (at 19.35 3.25 270) (size 1.288 1.288) (drill 0.78) (layers "*.Cu" "*.Mask") (remove_unused_layers no)
   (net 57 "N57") (solder_mask_margin 0.102))
  (pad "B31" thru_hole circle (at 20.35 1.25 270) (size 1.288 1.288) (drill 0.78) (layers "*.Cu" "*.Mask") (remove_unused_layers no)
   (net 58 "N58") (solder_mask_margin 0.102))
  (pad "B32" thru_hole circle (at 21.35 3.25 270) (size 1.288 1.288) (drill 0.78) (layers "*.Cu" "*.Mask") (remove_unused_layers no)
   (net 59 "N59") (solder_mask_margin 0.102)))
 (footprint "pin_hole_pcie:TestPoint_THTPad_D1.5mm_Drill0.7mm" (layer "F.Cu") (at 140.375 89.649397 180)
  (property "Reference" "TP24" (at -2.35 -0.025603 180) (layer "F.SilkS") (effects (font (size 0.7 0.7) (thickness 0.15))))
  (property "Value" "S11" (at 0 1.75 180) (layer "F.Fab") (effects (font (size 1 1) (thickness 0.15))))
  (pad "1" thru_hole circle (at 0 0 180) (size 1.5 1.5) (drill 0.7) (layers "*.Cu" "*.Mask") (remove_unused_layers no) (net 27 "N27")))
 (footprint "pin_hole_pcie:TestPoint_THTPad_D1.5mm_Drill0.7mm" (layer "F.Cu") (at 140.375 65.649397 180)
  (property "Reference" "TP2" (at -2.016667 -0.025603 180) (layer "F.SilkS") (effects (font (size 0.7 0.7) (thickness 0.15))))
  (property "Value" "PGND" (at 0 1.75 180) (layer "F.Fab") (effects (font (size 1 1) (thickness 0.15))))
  (pad "1" thru_hole circle (at 0 0 180) (size 1.5 1.5) (drill 0.7) (layers "*.Cu" "*.Mask") (remove_unused_layers no) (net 1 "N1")))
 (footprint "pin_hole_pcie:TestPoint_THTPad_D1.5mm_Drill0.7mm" (layer "F.Cu") (at 138.175 88.65 180)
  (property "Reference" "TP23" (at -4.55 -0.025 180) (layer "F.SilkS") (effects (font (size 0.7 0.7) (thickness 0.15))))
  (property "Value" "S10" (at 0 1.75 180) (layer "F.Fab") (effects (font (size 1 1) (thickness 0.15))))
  (pad "1" thru_hole circle (at 0 0 180) (size 1.5 1.5) (drill 0.7) (layers "*.Cu" "*.Mask") (remove_unused_layers no) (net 26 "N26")))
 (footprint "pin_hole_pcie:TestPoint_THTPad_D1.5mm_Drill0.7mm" (layer "F.Cu") (at 140.375 71.649397 180)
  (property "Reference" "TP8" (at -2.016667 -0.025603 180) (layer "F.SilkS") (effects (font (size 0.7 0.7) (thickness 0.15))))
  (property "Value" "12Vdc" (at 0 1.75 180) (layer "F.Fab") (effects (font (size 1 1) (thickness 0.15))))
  (pad "1" thru_hole circle (at 0 0 180) (size 1.5 1.5) (drill 0.7) (layers "*.Cu" "*.Mask") (remove_unused_layers no) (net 5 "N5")))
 (gr_rect (start 127.275 60.575) (end 144.2 101) (stroke (width 0.05) (type default)) (fill no) (layer "Edge.Cuts"))
 (segment (start 138.175 80.65) (end 133.9 80.65) (width 0.3) (layer "B.Cu") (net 14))
 (segment (start 135.900603 67.649397) (end 135.9 67.65) (width 0.3) (layer "B.Cu") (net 1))
 (segment (start 140.374397 65.65) (end 135.9 65.65) (width 0.3) (layer "B.Cu") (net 1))
 (segment (start 138.175 66.65) (end 133.9 66.65) (width 0.3) (layer "B.Cu") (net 1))
 (segment (start 140.375 67.649397) (end 135.900603 67.649397) (width 0.3) (layer "B.Cu") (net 1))
 (segment (start 138.175 68.65) (end 133.9 68.65) (width 0.3) (layer "B.Cu") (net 1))
 (segment (start 140.375 65.649397) (end 140.374397 65.65) (width 0.3) (layer "B.Cu") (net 1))
 (segment (start 140.374397 69.65) (end 135.9 69.65) (width 0.3) (layer "B.Cu") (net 9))
 (segment (start 140.375 69.649397) (end 140.374397 69.65) (width 0.3) (layer "B.Cu") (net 9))
 (segment (start 140.374397 95.65) (end 135.9 95.65) (width 0.3) (layer "B.Cu") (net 20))
 (segment (start 140.375 95.649397) (end 140.374397 95.65) (width 0.3) (layer "B.Cu") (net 20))
 (segment (start 138.175 70.65) (end 133.9 70.65) (width 0.3) (layer "B.Cu") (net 5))
 (segment (start 140.375 71.649397) (end 135.900603 71.649397) (width 0.3) (layer "B.Cu") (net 5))
 (segment (start 138.175 72.65) (end 133.9 72.65) (width 0.3) (layer "B.Cu") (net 5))
 (segment (start 135.900603 71.649397) (end 135.9 71.65) (width 0.3) (layer "B.Cu") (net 5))
 (segment (start 138.175 86.65) (end 133.9 86.65) (width 0.3) (layer "B.Cu") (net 6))
 (segment (start 138.175 78.65) (end 133.9 78.65) (width 0.3) (layer "B.Cu") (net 22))
 (segment (start 140.375 91.649397) (end 140.374397 91.65) (width 0.3) (layer "B.Cu") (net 3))
 (segment (start 140.374397 91.65) (end 135.9 91.65) (width 0.3) (layer "B.Cu") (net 3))
 (segment (start 140.374397 83.65) (end 135.9 83.65) (width 0.3) (layer "B.Cu") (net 18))
 (segment (start 140.375 83.649397) (end 140.374397 83.65) (width 0.3) (layer "B.Cu") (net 18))
 (segment (start 140.375 85.649397) (end 140.374397 85.65) (width 0.3) (layer "B.Cu") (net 4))
 (segment (start 140.374397 85.65) (end 135.9 85.65) (width 0.3) (layer "B.Cu") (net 4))
 (segment (start 138.175 90.65) (end 133.9 90.65) (width 0.3) (layer "B.Cu") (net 13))
 (segment (start 140.374397 81.65) (end 135.9 81.65) (width 0.3) (layer "B.Cu") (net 2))
 (segment (start 140.375 81.649397) (end 140.374397 81.65) (width 0.3) (layer "B.Cu") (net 2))
 (segment (start 133.9 94.65) (end 138.175 94.65) (width 0.3) (layer "B.Cu") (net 8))
 (segment (start 140.375 87.649397) (end 140.374397 87.65) (width 0.3) (layer "B.Cu") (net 21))
 (segment (start 140.374397 87.65) (end 135.9 87.65) (width 0.3) (layer "B.Cu") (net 21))
 (segment (start 140.375 73.649397) (end 140.374397 73.65) (width 0.3) (layer "B.Cu") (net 12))
 (segment (start 140.374397 73.65) (end 135.9 73.65) (width 0.3) (layer "B.Cu") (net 12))
 (segment (start 138.175 74.65) (end 133.9 74.65) (width 0.3) (layer "B.Cu") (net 24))
 (segment (start 138.175 82.65) (end 133.9 82.65) (width 0.3) (layer "B.Cu") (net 17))
 (segment (start 138.175 84.65) (end 133.9 84.65) (width 0.3) (layer "B.Cu") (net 23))
 (segment (start 133.9 96.65) (end 138.175 96.65) (width 0.3) (layer "B.Cu") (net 15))
 (segment (start 138.175 92.65) (end 133.9 92.65) (width 0.3) (layer "B.Cu") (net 7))
 (segment (start 135.900603 77.649397) (end 135.9 77.65) (width 0.3) (layer "B.Cu") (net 11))
 (segment (start 140.375 77.649397) (end 135.900603 77.649397) (width 0.3) (layer "B.Cu") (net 11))
 (segment (start 140.374397 79.65) (end 135.9 79.65) (width 0.3) (layer "B.Cu") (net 19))
 (segment (start 140.375 79.649397) (end 140.374397 79.65) (width 0.3) (layer "B.Cu") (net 19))
 (segment (start 140.374397 89.65) (end 135.9 89.65) (width 0.3) (layer "B.Cu") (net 27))
 (segment (start 140.375 89.649397) (end 140.374397 89.65) (width 0.3) (layer "B.Cu") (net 27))
 (segment (start 140.374397 97.65) (end 135.9 97.65) (width 0.3) (layer "B.Cu") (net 16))
 (segment (start 140.375 97.649397) (end 140.374397 97.65) (width 0.3) (layer "B.Cu") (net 16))
 (segment (start 138.175 64.65) (end 133.9 64.65) (width 0.3) (layer "B.Cu") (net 25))
 (segment (start 140.374397 93.65) (end 140.375 93.649397) (width 0.3) (layer "B.Cu") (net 10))
 (segment (start 135.9 93.65) (end 140.374397 93.65) (width 0.3) (layer "B.Cu") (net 10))
 (segment (start 138.175 88.65) (end 133.9 88.65) (width 0.3) (layer "B.Cu") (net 26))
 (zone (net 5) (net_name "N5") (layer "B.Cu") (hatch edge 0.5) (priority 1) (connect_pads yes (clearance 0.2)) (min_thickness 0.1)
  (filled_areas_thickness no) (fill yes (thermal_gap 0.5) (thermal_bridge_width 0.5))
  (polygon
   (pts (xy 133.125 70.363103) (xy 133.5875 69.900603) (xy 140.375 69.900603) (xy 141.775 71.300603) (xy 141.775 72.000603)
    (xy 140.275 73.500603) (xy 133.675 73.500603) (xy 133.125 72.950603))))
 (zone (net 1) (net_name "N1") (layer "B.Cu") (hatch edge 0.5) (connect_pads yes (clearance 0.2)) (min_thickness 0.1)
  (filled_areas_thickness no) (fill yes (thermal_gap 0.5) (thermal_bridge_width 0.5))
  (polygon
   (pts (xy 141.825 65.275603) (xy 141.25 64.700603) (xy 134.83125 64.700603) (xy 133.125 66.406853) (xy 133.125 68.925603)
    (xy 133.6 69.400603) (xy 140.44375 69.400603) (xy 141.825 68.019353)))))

